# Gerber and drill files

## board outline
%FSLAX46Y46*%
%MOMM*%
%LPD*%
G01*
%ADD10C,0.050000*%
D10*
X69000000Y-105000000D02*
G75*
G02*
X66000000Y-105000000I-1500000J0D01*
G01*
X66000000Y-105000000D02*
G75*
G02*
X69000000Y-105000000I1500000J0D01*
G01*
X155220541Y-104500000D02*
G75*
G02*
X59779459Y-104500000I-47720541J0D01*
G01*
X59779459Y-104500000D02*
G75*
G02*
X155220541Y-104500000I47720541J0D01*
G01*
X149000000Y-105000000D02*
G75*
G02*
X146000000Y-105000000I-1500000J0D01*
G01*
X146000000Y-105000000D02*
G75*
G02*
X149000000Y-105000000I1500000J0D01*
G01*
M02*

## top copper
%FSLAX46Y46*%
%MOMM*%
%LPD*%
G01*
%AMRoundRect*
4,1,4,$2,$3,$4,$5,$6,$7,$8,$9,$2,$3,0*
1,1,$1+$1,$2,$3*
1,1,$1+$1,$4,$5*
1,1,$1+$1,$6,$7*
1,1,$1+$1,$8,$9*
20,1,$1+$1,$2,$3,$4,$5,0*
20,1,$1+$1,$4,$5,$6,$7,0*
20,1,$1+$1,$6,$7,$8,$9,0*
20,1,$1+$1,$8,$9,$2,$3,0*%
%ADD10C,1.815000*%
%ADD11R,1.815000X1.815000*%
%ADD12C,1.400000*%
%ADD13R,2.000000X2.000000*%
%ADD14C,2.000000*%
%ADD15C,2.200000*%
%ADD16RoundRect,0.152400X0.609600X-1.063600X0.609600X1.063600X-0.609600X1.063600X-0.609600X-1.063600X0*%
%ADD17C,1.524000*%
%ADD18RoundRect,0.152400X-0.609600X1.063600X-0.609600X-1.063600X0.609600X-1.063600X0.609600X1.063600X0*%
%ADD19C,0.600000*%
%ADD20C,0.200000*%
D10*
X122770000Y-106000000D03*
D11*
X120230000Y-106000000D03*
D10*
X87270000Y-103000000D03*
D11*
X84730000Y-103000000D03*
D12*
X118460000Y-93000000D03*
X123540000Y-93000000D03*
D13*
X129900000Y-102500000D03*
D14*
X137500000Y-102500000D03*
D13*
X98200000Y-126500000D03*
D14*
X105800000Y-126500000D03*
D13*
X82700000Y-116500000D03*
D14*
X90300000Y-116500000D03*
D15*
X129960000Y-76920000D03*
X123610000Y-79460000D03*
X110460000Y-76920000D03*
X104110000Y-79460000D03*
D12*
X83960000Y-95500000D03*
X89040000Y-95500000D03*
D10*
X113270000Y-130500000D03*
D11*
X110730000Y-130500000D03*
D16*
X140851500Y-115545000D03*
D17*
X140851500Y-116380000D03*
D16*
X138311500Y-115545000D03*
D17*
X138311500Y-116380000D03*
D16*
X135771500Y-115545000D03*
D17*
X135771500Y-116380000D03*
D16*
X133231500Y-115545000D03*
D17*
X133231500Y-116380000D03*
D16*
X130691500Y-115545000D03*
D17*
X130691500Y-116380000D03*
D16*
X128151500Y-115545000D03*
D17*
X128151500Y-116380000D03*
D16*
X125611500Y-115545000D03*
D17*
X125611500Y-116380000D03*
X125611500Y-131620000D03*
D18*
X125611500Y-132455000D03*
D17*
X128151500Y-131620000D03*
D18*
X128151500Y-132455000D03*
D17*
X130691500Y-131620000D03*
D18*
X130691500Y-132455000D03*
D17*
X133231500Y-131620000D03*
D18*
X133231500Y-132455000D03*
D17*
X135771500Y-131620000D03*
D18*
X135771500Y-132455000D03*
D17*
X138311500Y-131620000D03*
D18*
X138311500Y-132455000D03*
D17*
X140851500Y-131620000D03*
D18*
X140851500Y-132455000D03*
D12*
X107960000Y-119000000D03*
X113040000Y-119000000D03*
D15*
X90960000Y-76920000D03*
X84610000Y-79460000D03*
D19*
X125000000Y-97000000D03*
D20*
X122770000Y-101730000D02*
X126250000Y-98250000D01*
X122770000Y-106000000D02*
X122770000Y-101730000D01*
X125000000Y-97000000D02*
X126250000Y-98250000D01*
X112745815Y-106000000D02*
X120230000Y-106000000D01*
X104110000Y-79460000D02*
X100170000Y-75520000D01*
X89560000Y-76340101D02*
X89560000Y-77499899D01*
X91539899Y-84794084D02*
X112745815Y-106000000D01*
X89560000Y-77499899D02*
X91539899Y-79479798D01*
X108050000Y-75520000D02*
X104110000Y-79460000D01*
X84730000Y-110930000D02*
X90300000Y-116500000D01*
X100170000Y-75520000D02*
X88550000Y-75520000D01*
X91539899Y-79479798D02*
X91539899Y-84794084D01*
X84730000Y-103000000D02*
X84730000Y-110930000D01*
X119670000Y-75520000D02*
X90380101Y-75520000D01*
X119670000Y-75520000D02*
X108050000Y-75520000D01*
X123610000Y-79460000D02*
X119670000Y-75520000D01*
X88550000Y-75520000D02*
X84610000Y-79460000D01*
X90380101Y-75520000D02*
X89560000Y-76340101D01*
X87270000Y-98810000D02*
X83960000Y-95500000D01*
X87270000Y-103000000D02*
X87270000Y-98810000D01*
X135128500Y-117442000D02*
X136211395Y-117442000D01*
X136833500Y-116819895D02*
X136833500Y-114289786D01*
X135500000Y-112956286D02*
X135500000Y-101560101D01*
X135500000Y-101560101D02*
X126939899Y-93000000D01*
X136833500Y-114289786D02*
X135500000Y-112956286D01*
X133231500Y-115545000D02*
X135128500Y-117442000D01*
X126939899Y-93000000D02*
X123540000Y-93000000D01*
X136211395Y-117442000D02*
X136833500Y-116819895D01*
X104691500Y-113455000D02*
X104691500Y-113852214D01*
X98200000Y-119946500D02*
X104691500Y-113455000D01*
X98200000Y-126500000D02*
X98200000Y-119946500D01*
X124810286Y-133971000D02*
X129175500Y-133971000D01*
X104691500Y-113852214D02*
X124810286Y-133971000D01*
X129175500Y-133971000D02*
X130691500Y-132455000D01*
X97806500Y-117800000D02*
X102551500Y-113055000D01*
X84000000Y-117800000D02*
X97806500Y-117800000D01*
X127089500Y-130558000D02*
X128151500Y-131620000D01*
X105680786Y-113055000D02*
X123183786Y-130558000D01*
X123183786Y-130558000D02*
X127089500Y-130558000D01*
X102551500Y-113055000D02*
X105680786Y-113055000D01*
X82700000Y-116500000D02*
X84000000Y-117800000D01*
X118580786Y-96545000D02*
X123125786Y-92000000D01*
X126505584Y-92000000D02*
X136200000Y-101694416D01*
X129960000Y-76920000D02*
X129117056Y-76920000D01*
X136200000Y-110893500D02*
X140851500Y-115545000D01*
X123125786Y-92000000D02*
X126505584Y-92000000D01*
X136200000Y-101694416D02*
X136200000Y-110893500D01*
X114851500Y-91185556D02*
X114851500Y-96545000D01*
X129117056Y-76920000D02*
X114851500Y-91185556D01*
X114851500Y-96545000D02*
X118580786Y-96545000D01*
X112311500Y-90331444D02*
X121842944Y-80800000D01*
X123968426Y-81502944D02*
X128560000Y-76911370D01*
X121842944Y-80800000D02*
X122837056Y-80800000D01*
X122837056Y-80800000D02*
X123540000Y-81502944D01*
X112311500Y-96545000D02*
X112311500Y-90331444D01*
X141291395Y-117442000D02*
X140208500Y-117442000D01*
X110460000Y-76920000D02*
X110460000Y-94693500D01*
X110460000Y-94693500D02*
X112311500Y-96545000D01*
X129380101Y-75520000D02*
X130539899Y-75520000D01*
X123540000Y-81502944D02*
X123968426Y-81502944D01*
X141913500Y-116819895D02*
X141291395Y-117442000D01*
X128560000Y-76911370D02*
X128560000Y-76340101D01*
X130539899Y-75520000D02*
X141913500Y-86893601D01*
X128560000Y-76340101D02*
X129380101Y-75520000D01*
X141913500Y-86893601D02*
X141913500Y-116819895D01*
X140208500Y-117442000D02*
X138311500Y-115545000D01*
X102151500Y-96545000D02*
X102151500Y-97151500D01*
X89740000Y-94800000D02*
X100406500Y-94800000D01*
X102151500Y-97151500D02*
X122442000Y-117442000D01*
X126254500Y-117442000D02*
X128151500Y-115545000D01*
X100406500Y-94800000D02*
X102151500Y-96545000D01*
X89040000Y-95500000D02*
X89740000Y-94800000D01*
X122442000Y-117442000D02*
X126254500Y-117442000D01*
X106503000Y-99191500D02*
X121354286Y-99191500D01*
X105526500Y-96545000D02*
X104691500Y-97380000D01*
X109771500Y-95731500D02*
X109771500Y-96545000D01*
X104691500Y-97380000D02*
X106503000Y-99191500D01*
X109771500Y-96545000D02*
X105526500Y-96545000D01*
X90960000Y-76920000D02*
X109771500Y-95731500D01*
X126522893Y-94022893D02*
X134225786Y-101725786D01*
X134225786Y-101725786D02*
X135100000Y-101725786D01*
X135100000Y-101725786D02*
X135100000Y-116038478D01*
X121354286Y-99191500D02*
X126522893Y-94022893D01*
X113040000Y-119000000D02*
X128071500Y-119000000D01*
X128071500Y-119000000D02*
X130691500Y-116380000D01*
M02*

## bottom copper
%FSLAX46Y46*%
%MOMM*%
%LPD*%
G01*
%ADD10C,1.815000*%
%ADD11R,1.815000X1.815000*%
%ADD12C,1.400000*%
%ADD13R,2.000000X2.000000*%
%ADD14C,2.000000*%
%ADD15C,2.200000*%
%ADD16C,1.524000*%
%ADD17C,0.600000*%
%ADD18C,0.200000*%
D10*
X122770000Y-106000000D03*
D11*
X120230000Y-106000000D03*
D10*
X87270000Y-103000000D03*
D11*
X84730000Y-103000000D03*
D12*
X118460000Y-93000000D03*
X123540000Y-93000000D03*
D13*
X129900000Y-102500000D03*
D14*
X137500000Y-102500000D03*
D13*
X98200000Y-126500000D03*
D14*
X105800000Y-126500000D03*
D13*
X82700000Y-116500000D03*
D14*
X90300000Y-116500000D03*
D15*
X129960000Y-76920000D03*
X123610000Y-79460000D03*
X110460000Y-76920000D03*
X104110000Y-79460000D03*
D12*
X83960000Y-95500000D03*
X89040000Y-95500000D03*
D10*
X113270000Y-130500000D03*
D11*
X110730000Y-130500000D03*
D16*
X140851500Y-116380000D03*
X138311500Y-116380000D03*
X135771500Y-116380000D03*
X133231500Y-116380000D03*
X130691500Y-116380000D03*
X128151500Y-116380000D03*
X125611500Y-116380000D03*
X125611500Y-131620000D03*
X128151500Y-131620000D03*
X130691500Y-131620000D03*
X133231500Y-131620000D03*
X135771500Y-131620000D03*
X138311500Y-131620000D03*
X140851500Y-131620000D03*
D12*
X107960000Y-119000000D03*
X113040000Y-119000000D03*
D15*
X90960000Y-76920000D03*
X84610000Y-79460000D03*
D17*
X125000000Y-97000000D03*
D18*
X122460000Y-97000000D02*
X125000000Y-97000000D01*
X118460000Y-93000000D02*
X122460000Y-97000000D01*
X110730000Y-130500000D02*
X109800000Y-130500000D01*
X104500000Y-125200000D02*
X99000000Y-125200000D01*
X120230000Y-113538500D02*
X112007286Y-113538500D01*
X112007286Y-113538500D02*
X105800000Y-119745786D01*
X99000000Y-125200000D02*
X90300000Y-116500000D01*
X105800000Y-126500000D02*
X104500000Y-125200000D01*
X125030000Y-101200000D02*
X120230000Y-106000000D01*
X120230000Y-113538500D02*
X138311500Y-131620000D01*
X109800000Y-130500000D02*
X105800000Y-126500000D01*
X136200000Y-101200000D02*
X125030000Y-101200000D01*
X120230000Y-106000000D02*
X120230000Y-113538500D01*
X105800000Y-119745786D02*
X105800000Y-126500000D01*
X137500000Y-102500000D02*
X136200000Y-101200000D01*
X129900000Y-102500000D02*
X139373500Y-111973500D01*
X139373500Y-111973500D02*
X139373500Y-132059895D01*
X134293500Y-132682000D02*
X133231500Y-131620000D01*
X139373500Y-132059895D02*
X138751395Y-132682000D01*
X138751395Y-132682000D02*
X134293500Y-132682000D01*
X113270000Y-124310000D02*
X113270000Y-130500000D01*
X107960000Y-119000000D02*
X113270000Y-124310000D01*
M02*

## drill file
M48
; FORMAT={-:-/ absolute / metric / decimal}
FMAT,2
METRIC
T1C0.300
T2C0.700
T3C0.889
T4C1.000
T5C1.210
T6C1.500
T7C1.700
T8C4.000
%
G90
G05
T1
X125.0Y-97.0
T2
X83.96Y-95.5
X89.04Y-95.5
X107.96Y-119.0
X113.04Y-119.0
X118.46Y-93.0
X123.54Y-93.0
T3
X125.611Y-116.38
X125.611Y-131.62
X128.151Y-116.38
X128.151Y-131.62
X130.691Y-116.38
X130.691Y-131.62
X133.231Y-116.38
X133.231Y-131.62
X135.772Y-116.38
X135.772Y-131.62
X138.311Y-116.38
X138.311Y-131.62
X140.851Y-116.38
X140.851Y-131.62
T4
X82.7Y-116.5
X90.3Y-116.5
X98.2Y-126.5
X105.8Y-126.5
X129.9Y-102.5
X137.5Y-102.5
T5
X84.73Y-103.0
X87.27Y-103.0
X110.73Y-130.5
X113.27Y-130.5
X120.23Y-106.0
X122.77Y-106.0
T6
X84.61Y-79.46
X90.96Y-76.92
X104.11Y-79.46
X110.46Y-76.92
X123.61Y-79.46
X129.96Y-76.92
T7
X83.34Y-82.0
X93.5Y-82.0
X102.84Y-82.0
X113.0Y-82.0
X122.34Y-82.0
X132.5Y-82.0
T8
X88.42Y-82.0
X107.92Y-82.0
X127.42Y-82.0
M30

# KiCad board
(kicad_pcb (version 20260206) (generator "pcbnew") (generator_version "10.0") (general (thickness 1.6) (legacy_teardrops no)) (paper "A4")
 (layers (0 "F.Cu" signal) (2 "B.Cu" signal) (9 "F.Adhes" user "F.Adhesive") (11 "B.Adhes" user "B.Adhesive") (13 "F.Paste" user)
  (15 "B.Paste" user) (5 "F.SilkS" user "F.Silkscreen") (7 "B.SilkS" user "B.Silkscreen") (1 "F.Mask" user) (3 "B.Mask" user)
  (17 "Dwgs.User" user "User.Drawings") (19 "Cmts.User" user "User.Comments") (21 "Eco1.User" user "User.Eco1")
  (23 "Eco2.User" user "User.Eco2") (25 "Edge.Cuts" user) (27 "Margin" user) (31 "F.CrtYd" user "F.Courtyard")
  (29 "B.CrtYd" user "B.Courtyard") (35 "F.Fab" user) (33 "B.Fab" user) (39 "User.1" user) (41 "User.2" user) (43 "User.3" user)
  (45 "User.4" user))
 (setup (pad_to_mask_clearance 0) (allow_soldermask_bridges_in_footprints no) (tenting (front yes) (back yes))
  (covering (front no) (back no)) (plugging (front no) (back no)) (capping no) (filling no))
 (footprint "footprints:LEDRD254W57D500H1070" (layer "F.Cu") (at 121.5 106)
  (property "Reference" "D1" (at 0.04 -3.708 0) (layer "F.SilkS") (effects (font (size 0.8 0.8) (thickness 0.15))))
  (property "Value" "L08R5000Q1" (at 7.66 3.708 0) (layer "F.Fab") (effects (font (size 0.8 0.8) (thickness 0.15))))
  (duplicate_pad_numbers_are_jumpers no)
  (pad "A" thru_hole circle (at 1.27 0) (size 1.815 1.815) (drill 1.21) (layers "*.Cu" "*.Mask") (remove_unused_layers no)
   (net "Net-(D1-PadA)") (solder_mask_margin 0.102))
  (pad "C" thru_hole rect (at -1.27 0) (size 1.815 1.815) (drill 1.21) (layers "*.Cu" "*.Mask") (remove_unused_layers no) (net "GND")
   (solder_mask_margin 0.102)))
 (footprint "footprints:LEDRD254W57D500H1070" (layer "F.Cu") (at 86 103)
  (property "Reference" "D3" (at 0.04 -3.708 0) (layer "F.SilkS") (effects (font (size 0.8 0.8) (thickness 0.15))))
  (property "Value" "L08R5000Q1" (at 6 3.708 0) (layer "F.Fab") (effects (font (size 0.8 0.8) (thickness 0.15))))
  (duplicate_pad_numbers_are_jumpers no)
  (pad "A" thru_hole circle (at 1.27 0) (size 1.815 1.815) (drill 1.21) (layers "*.Cu" "*.Mask") (remove_unused_layers no)
   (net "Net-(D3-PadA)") (solder_mask_margin 0.102))
  (pad "C" thru_hole rect (at -1.27 0) (size 1.815 1.815) (drill 1.21) (layers "*.Cu" "*.Mask") (remove_unused_layers no) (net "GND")
   (solder_mask_margin 0.102)))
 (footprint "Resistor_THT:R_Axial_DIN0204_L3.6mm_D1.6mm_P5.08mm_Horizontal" (layer "F.Cu") (at 118.46 93)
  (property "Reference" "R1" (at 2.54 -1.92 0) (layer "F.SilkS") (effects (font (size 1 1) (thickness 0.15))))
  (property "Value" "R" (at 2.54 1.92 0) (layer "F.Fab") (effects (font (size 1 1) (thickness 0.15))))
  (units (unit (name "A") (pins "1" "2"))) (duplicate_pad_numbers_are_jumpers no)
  (pad "1" thru_hole circle (at 0 0) (size 1.4 1.4) (drill 0.7) (layers "*.Cu" "*.Mask") (remove_unused_layers no) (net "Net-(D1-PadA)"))
  (pad "2" thru_hole circle (at 5.08 0) (size 1.4 1.4) (drill 0.7) (layers "*.Cu" "*.Mask") (remove_unused_layers no)
   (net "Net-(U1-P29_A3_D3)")))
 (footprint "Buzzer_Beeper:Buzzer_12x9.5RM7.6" (layer "F.Cu") (at 129.9 102.5)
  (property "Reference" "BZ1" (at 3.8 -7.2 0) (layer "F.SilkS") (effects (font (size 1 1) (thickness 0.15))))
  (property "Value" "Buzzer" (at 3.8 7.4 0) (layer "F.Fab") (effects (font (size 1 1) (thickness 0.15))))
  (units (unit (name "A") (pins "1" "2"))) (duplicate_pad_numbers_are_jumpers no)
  (pad "1" thru_hole rect (at 0 0) (size 2 2) (drill 1) (layers "*.Cu" "*.Mask") (remove_unused_layers no) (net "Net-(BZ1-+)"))
  (pad "2" thru_hole circle (at 7.6 0) (size 2 2) (drill 1) (layers "*.Cu" "*.Mask") (remove_unused_layers no) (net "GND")))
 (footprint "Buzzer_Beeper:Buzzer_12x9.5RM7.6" (layer "F.Cu") (at 98.2 126.5)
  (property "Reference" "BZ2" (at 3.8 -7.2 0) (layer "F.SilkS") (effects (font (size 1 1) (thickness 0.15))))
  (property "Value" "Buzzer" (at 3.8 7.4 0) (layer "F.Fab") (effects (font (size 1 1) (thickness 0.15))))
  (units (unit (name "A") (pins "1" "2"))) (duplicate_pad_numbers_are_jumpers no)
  (pad "1" thru_hole rect (at 0 0) (size 2 2) (drill 1) (layers "*.Cu" "*.Mask") (remove_unused_layers no) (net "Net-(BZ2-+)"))
  (pad "2" thru_hole circle (at 7.6 0) (size 2 2) (drill 1) (layers "*.Cu" "*.Mask") (remove_unused_layers no) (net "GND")))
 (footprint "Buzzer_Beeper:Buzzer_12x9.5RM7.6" (layer "F.Cu") (at 82.7 116.5)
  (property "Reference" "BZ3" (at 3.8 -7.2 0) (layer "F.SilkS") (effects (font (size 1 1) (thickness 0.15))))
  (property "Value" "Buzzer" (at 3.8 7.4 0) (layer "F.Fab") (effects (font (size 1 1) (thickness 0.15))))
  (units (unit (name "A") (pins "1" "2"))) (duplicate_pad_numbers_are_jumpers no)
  (pad "1" thru_hole rect (at 0 0) (size 2 2) (drill 1) (layers "*.Cu" "*.Mask") (remove_unused_layers no) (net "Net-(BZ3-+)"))
  (pad "2" thru_hole circle (at 7.6 0) (size 2 2) (drill 1) (layers "*.Cu" "*.Mask") (remove_unused_layers no) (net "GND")))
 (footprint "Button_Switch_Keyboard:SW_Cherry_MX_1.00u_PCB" (layer "F.Cu") (at 129.96 76.92)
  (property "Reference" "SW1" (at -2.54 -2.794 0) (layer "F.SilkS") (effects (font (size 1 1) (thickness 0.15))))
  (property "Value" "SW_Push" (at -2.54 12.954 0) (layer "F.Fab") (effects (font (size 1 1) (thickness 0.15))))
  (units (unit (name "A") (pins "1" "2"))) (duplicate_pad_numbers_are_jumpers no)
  (pad "" np_thru_hole circle (at -7.62 5.08) (size 1.7 1.7) (drill 1.7) (layers "*.Cu" "*.Mask"))
  (pad "" np_thru_hole circle (at -2.54 5.08) (size 4 4) (drill 4) (layers "*.Cu" "*.Mask"))
  (pad "" np_thru_hole circle (at 2.54 5.08) (size 1.7 1.7) (drill 1.7) (layers "*.Cu" "*.Mask"))
  (pad "1" thru_hole circle (at 0 0) (size 2.2 2.2) (drill 1.5) (layers "*.Cu" "*.Mask") (remove_unused_layers no)
   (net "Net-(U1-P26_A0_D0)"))
  (pad "2" thru_hole circle (at -6.35 2.54) (size 2.2 2.2) (drill 1.5) (layers "*.Cu" "*.Mask") (remove_unused_layers no) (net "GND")))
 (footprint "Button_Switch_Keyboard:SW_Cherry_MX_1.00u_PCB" (layer "F.Cu") (at 110.46 76.92)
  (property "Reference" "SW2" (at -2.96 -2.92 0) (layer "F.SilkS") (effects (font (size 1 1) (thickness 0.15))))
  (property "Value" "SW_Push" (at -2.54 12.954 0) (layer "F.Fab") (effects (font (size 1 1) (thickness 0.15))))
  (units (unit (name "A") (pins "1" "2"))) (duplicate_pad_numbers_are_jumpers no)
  (pad "" np_thru_hole circle (at -7.62 5.08) (size 1.7 1.7) (drill 1.7) (layers "*.Cu" "*.Mask"))
  (pad "" np_thru_hole circle (at -2.54 5.08) (size 4 4) (drill 4) (layers "*.Cu" "*.Mask"))
  (pad "" np_thru_hole circle (at 2.54 5.08) (size 1.7 1.7) (drill 1.7) (layers "*.Cu" "*.Mask"))
  (pad "1" thru_hole circle (at 0 0) (size 2.2 2.2) (drill 1.5) (layers "*.Cu" "*.Mask") (remove_unused_layers no)
   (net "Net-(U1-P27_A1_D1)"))
  (pad "2" thru_hole circle (at -6.35 2.54) (size 2.2 2.2) (drill 1.5) (layers "*.Cu" "*.Mask") (remove_unused_layers no) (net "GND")))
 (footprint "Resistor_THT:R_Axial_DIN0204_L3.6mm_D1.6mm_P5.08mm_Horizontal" (layer "F.Cu") (at 83.96 95.5)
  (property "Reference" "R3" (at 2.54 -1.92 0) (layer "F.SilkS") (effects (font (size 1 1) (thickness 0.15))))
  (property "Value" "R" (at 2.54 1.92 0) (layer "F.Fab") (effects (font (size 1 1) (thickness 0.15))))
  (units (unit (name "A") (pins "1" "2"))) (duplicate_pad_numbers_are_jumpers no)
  (pad "1" thru_hole circle (at 0 0) (size 1.4 1.4) (drill 0.7) (layers "*.Cu" "*.Mask") (remove_unused_layers no) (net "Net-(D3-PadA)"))
  (pad "2" thru_hole circle (at 5.08 0) (size 1.4 1.4) (drill 0.7) (layers "*.Cu" "*.Mask") (remove_unused_layers no)
   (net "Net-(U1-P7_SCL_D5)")))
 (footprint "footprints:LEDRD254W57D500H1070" (layer "F.Cu") (at 112 130.5)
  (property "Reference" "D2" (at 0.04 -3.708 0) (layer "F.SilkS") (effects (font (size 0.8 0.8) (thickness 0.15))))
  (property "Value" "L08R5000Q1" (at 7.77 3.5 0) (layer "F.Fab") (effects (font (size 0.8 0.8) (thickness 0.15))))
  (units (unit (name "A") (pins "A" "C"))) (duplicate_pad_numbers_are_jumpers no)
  (pad "A" thru_hole circle (at 1.27 0) (size 1.815 1.815) (drill 1.21) (layers "*.Cu" "*.Mask") (remove_unused_layers no)
   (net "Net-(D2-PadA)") (solder_mask_margin 0.102))
  (pad "C" thru_hole rect (at -1.27 0) (size 1.815 1.815) (drill 1.21) (layers "*.Cu" "*.Mask") (remove_unused_layers no) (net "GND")
   (solder_mask_margin 0.102)))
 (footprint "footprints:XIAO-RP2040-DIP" (layer "F.Cu") (at 133.2315 124)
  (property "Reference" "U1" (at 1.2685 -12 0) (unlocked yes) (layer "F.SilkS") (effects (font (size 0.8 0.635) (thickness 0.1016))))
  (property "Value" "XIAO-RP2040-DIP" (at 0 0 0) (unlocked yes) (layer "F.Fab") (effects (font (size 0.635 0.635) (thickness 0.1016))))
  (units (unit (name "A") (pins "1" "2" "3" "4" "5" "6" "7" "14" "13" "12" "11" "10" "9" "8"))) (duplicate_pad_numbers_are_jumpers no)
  (pad "1" smd roundrect (at 7.62 -8.455 90) (size 2.432 1.524) (layers "F.Cu" "F.Mask") (roundrect_rratio 0.1) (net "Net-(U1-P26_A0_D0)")
   (thermal_bridge_angle 45))
  (pad "1" thru_hole circle (at 7.62 -7.62 90) (size 1.524 1.524) (drill 0.889) (layers "*.Cu" "*.Mask") (remove_unused_layers no)
   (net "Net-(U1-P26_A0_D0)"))
  (pad "2" smd roundrect (at 5.08 -8.455 90) (size 2.432 1.524) (layers "F.Cu" "F.Mask") (roundrect_rratio 0.1) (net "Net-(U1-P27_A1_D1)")
   (thermal_bridge_angle 45))
  (pad "2" thru_hole circle (at 5.08 -7.62 90) (size 1.524 1.524) (drill 0.889) (layers "*.Cu" "*.Mask") (remove_unused_layers no)
   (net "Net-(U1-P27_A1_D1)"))
  (pad "3" smd roundrect (at 2.54 -8.455 90) (size 2.432 1.524) (layers "F.Cu" "F.Mask") (roundrect_rratio 0.1) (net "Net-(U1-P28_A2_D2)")
   (thermal_bridge_angle 45))
  (pad "3" thru_hole circle (at 2.54 -7.62 90) (size 1.524 1.524) (drill 0.889) (layers "*.Cu" "*.Mask") (remove_unused_layers no)
   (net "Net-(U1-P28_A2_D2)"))
  (pad "4" smd roundrect (at 0 -8.455 90) (size 2.432 1.524) (layers "F.Cu" "F.Mask") (roundrect_rratio 0.1) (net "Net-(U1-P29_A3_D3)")
   (thermal_bridge_angle 45))
  (pad "4" thru_hole circle (at 0 -7.62 90) (size 1.524 1.524) (drill 0.889) (layers "*.Cu" "*.Mask") (remove_unused_layers no)
   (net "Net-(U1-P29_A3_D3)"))
  (pad "5" smd roundrect (at -2.54 -8.455 90) (size 2.432 1.524) (layers "F.Cu" "F.Mask") (roundrect_rratio 0.1) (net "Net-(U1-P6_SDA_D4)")
   (thermal_bridge_angle 45))
  (pad "5" thru_hole circle (at -2.54 -7.62 90) (size 1.524 1.524) (drill 0.889) (layers "*.Cu" "*.Mask") (remove_unused_layers no)
   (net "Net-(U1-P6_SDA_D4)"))
  (pad "6" smd roundrect (at -5.08 -8.455 90) (size 2.432 1.524) (layers "F.Cu" "F.Mask") (roundrect_rratio 0.1) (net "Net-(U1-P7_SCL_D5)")
   (thermal_bridge_angle 45))
  (pad "6" thru_hole circle (at -5.08 -7.62 90) (size 1.524 1.524) (drill 0.889) (layers "*.Cu" "*.Mask") (remove_unused_layers no)
   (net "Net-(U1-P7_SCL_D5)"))
  (pad "7" smd roundrect (at -7.62 -8.455 90) (size 2.432 1.524) (layers "F.Cu" "F.Mask") (roundrect_rratio 0.1)
   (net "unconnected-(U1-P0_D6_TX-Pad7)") (thermal_bridge_angle 45))
  (pad "7" thru_hole circle (at -7.62 -7.62 90) (size 1.524 1.524) (drill 0.889) (layers "*.Cu" "*.Mask") (remove_unused_layers no)
   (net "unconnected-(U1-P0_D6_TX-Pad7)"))
  (pad "8" thru_hole circle (at -7.62 7.62 270) (size 1.524 1.524) (drill 0.889) (layers "*.Cu" "*.Mask") (remove_unused_layers no)
   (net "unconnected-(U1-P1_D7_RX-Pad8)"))
  (pad "8" smd roundrect (at -7.62 8.455 270) (size 2.432 1.524) (layers "F.Cu" "F.Mask") (roundrect_rratio 0.1)
   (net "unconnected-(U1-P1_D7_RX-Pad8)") (thermal_bridge_angle 45))
  (pad "9" thru_hole circle (at -5.08 7.62 270) (size 1.524 1.524) (drill 0.889) (layers "*.Cu" "*.Mask") (remove_unused_layers no)
   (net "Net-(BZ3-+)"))
  (pad "9" smd roundrect (at -5.08 8.455 270) (size 2.432 1.524) (layers "F.Cu" "F.Mask") (roundrect_rratio 0.1) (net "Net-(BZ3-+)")
   (thermal_bridge_angle 45))
  (pad "10" thru_hole circle (at -2.54 7.62 270) (size 1.524 1.524) (drill 0.889) (layers "*.Cu" "*.Mask") (remove_unused_layers no)
   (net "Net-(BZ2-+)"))
  (pad "10" smd roundrect (at -2.54 8.455 270) (size 2.432 1.524) (layers "F.Cu" "F.Mask") (roundrect_rratio 0.1) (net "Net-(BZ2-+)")
   (thermal_bridge_angle 45))
  (pad "11" thru_hole circle (at 0 7.62 270) (size 1.524 1.524) (drill 0.889) (layers "*.Cu" "*.Mask") (remove_unused_layers no)
   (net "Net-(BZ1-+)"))
  (pad "11" smd roundrect (at 0 8.455 270) (size 2.432 1.524) (layers "F.Cu" "F.Mask") (roundrect_rratio 0.1) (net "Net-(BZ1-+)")
   (thermal_bridge_angle 45))
  (pad "12" thru_hole circle (at 2.54 7.62 270) (size 1.524 1.524) (drill 0.889) (layers "*.Cu" "*.Mask") (remove_unused_layers no)
   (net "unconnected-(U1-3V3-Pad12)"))
  (pad "12" smd roundrect (at 2.54 8.455 270) (size 2.432 1.524) (layers "F.Cu" "F.Mask") (roundrect_rratio 0.1)
   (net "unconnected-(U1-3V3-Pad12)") (thermal_bridge_angle 45))
  (pad "13" thru_hole circle (at 5.08 7.62 270) (size 1.524 1.524) (drill 0.889) (layers "*.Cu" "*.Mask") (remove_unused_layers no)
   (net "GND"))
  (pad "13" smd roundrect (at 5.08 8.455 270) (size 2.432 1.524) (layers "F.Cu" "F.Mask") (roundrect_rratio 0.1) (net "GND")
   (thermal_bridge_angle 45))
  (pad "14" thru_hole circle (at 7.62 7.62 270) (size 1.524 1.524) (drill 0.889) (layers "*.Cu" "*.Mask") (remove_unused_layers no)
   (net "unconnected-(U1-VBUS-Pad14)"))
  (pad "14" smd roundrect (at 7.62 8.455 270) (size 2.432 1.524) (layers "F.Cu" "F.Mask") (roundrect_rratio 0.1)
   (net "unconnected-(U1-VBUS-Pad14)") (thermal_bridge_angle 45)))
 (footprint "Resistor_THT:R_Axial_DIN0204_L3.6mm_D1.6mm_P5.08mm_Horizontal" (layer "F.Cu") (at 107.96 119)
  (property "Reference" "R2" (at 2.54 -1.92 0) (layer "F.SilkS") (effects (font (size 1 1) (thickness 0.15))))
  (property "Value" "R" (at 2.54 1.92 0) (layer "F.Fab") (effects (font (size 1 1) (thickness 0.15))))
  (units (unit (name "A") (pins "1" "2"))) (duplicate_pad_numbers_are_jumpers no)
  (pad "1" thru_hole circle (at 0 0) (size 1.4 1.4) (drill 0.7) (layers "*.Cu" "*.Mask") (remove_unused_layers no) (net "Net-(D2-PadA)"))
  (pad "2" thru_hole circle (at 5.08 0) (size 1.4 1.4) (drill 0.7) (layers "*.Cu" "*.Mask") (remove_unused_layers no)
   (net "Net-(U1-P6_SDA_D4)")))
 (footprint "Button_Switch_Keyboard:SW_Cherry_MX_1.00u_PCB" (layer "F.Cu") (at 90.96 76.92)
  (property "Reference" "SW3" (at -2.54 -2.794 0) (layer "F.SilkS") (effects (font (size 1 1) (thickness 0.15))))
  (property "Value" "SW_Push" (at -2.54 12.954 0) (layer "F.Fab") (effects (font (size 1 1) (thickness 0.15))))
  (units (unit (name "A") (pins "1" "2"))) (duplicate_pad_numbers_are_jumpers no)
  (pad "" np_thru_hole circle (at -7.62 5.08) (size 1.7 1.7) (drill 1.7) (layers "*.Cu" "*.Mask"))
  (pad "" np_thru_hole circle (at -2.54 5.08) (size 4 4) (drill 4) (layers "*.Cu" "*.Mask"))
  (pad "" np_thru_hole circle (at 2.54 5.08) (size 1.7 1.7) (drill 1.7) (layers "*.Cu" "*.Mask"))
  (pad "1" thru_hole circle (at 0 0) (size 2.2 2.2) (drill 1.5) (layers "*.Cu" "*.Mask") (remove_unused_layers no)
   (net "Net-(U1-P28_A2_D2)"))
  (pad "2" thru_hole circle (at -6.35 2.54) (size 2.2 2.2) (drill 1.5) (layers "*.Cu" "*.Mask") (remove_unused_layers no) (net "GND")))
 (gr_circle (center 67.5 105) (end 66 105) (stroke (width 0.05) (type default)) (fill no) (layer "Edge.Cuts"))
 (gr_circle (center 107.5 104.5) (end 80 65.5) (stroke (width 0.05) (type default)) (fill no) (layer "Edge.Cuts"))
 (gr_circle (center 147.5 105) (end 149 105) (stroke (width 0.05) (type default)) (fill no) (layer "Edge.Cuts"))
 (segment (start 122.77 101.73) (end 126.25 98.25) (width 0.2) (layer "F.Cu") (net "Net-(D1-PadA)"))
 (segment (start 122.77 106) (end 122.77 101.73) (width 0.2) (layer "F.Cu") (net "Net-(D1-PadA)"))
 (segment (start 125 97) (end 126.25 98.25) (width 0.2) (layer "F.Cu") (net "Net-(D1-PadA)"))
 (via (at 125 97) (size 0.6) (drill 0.3) (layers "F.Cu" "B.Cu") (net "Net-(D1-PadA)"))
 (segment (start 122.46 97) (end 125 97) (width 0.2) (layer "B.Cu") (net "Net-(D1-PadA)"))
 (segment (start 118.46 93) (end 122.46 97) (width 0.2) (layer "B.Cu") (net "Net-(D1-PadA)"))
 (segment (start 112.745815 106) (end 120.23 106) (width 0.2) (layer "F.Cu") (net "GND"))
 (segment (start 104.11 79.46) (end 100.17 75.52) (width 0.2) (layer "F.Cu") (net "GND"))
 (segment (start 89.56 76.340101) (end 89.56 77.499899) (width 0.2) (layer "F.Cu") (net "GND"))
 (segment (start 91.539899 84.794084) (end 112.745815 106) (width 0.2) (layer "F.Cu") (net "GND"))
 (segment (start 89.56 77.499899) (end 91.539899 79.479798) (width 0.2) (layer "F.Cu") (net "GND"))
 (segment (start 108.05 75.52) (end 104.11 79.46) (width 0.2) (layer "F.Cu") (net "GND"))
 (segment (start 84.73 110.93) (end 90.3 116.5) (width 0.2) (layer "F.Cu") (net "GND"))
 (segment (start 100.17 75.52) (end 88.55 75.52) (width 0.2) (layer "F.Cu") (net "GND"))
 (segment (start 91.539899 79.479798) (end 91.539899 84.794084) (width 0.2) (layer "F.Cu") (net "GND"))
 (segment (start 84.73 103) (end 84.73 110.93) (width 0.2) (layer "F.Cu") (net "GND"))
 (segment (start 119.67 75.52) (end 90.380101 75.52) (width 0.2) (layer "F.Cu") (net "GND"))
 (segment (start 119.67 75.52) (end 108.05 75.52) (width 0.2) (layer "F.Cu") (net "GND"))
 (segment (start 123.61 79.46) (end 119.67 75.52) (width 0.2) (layer "F.Cu") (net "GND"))
 (segment (start 88.55 75.52) (end 84.61 79.46) (width 0.2) (layer "F.Cu") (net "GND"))
 (segment (start 90.380101 75.52) (end 89.56 76.340101) (width 0.2) (layer "F.Cu") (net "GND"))
 (segment (start 110.73 130.5) (end 109.8 130.5) (width 0.2) (layer "B.Cu") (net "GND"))
 (segment (start 104.5 125.2) (end 99 125.2) (width 0.2) (layer "B.Cu") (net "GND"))
 (segment (start 120.23 113.5385) (end 112.007286 113.5385) (width 0.2) (layer "B.Cu") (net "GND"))
 (segment (start 112.007286 113.5385) (end 105.8 119.745786) (width 0.2) (layer "B.Cu") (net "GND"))
 (segment (start 99 125.2) (end 90.3 116.5) (width 0.2) (layer "B.Cu") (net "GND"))
 (segment (start 105.8 126.5) (end 104.5 125.2) (width 0.2) (layer "B.Cu") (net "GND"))
 (segment (start 125.03 101.2) (end 120.23 106) (width 0.2) (layer "B.Cu") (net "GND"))
 (segment (start 120.23 113.5385) (end 138.3115 131.62) (width 0.2) (layer "B.Cu") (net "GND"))
 (segment (start 109.8 130.5) (end 105.8 126.5) (width 0.2) (layer "B.Cu") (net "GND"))
 (segment (start 136.2 101.2) (end 125.03 101.2) (width 0.2) (layer "B.Cu") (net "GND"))
 (segment (start 120.23 106) (end 120.23 113.5385) (width 0.2) (layer "B.Cu") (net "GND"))
 (segment (start 105.8 119.745786) (end 105.8 126.5) (width 0.2) (layer "B.Cu") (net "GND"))
 (segment (start 137.5 102.5) (end 136.2 101.2) (width 0.2) (layer "B.Cu") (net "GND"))
 (segment (start 87.27 98.81) (end 83.96 95.5) (width 0.2) (layer "F.Cu") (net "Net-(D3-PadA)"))
 (segment (start 87.27 103) (end 87.27 98.81) (width 0.2) (layer "F.Cu") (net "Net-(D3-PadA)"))
 (segment (start 135.1285 117.442) (end 136.211395 117.442) (width 0.2) (layer "F.Cu") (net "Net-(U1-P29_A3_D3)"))
 (segment (start 136.8335 116.819895) (end 136.8335 114.289786) (width 0.2) (layer "F.Cu") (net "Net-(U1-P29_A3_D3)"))
 (segment (start 135.5 112.956286) (end 135.5 101.560101) (width 0.2) (layer "F.Cu") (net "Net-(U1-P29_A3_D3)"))
 (segment (start 135.5 101.560101) (end 126.939899 93) (width 0.2) (layer "F.Cu") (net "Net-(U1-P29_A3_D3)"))
 (segment (start 136.8335 114.289786) (end 135.5 112.956286) (width 0.2) (layer "F.Cu") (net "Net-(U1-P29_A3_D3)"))
 (segment (start 133.2315 115.545) (end 135.1285 117.442) (width 0.2) (layer "F.Cu") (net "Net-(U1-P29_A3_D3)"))
 (segment (start 126.939899 93) (end 123.54 93) (width 0.2) (layer "F.Cu") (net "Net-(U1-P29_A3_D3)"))
 (segment (start 136.211395 117.442) (end 136.8335 116.819895) (width 0.2) (layer "F.Cu") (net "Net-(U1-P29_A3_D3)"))
 (segment (start 129.9 102.5) (end 139.3735 111.9735) (width 0.2) (layer "B.Cu") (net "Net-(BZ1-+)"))
 (segment (start 139.3735 111.9735) (end 139.3735 132.059895) (width 0.2) (layer "B.Cu") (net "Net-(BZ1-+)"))
 (segment (start 134.2935 132.682) (end 133.2315 131.62) (width 0.2) (layer "B.Cu") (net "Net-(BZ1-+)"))
 (segment (start 139.3735 132.059895) (end 138.751395 132.682) (width 0.2) (layer "B.Cu") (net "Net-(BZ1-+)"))
 (segment (start 138.751395 132.682) (end 134.2935 132.682) (width 0.2) (layer "B.Cu") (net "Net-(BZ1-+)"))
 (segment (start 104.6915 113.455) (end 104.6915 113.852214) (width 0.2) (layer "F.Cu") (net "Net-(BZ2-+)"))
 (segment (start 98.2 119.9465) (end 104.6915 113.455) (width 0.2) (layer "F.Cu") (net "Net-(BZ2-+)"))
 (segment (start 98.2 126.5) (end 98.2 119.9465) (width 0.2) (layer "F.Cu") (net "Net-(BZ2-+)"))
 (segment (start 124.810286 133.971) (end 129.1755 133.971) (width 0.2) (layer "F.Cu") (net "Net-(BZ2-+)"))
 (segment (start 104.6915 113.852214) (end 124.810286 133.971) (width 0.2) (layer "F.Cu") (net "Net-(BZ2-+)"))
 (segment (start 129.1755 133.971) (end 130.6915 132.455) (width 0.2) (layer "F.Cu") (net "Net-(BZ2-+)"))
 (segment (start 97.8065 117.8) (end 102.5515 113.055) (width 0.2) (layer "F.Cu") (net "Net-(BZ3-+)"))
 (segment (start 84 117.8) (end 97.8065 117.8) (width 0.2) (layer "F.Cu") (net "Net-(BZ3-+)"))
 (segment (start 127.0895 130.558) (end 128.1515 131.62) (width 0.2) (layer "F.Cu") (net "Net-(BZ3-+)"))
 (segment (start 105.680786 113.055) (end 123.183786 130.558) (width 0.2) (layer "F.Cu") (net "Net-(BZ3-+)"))
 (segment (start 123.183786 130.558) (end 127.0895 130.558) (width 0.2) (layer "F.Cu") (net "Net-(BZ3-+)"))
 (segment (start 102.5515 113.055) (end 105.680786 113.055) (width 0.2) (layer "F.Cu") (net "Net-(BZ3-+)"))
 (segment (start 82.7 116.5) (end 84 117.8) (width 0.2) (layer "F.Cu") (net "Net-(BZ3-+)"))
 (segment (start 118.580786 96.545) (end 123.125786 92) (width 0.2) (layer "F.Cu") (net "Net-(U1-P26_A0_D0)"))
 (segment (start 126.505584 92) (end 136.2 101.694416) (width 0.2) (layer "F.Cu") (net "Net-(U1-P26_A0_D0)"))
 (segment (start 129.96 76.92) (end 129.117056 76.92) (width 0.2) (layer "F.Cu") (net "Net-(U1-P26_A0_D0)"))
 (segment (start 136.2 110.8935) (end 140.8515 115.545) (width 0.2) (layer "F.Cu") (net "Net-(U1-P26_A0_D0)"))
 (segment (start 123.125786 92) (end 126.505584 92) (width 0.2) (layer "F.Cu") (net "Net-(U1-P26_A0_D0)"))
 (segment (start 136.2 101.694416) (end 136.2 110.8935) (width 0.2) (layer "F.Cu") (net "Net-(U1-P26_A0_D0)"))
 (segment (start 114.8515 91.185556) (end 114.8515 96.545) (width 0.2) (layer "F.Cu") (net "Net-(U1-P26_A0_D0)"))
 (segment (start 129.117056 76.92) (end 114.8515 91.185556) (width 0.2) (layer "F.Cu") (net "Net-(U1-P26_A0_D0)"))
 (segment (start 114.8515 96.545) (end 118.580786 96.545) (width 0.2) (layer "F.Cu") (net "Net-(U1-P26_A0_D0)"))
 (segment (start 112.3115 90.331444) (end 121.842944 80.8) (width 0.2) (layer "F.Cu") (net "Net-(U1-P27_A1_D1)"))
 (segment (start 123.968426 81.502944) (end 128.56 76.91137) (width 0.2) (layer "F.Cu") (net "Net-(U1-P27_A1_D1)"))
 (segment (start 121.842944 80.8) (end 122.837056 80.8) (width 0.2) (layer "F.Cu") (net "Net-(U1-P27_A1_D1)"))
 (segment (start 122.837056 80.8) (end 123.54 81.502944) (width 0.2) (layer "F.Cu") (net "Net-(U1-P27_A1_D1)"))
 (segment (start 112.3115 96.545) (end 112.3115 90.331444) (width 0.2) (layer "F.Cu") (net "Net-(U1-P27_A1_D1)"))
 (segment (start 141.291395 117.442) (end 140.2085 117.442) (width 0.2) (layer "F.Cu") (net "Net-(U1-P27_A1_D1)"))
 (segment (start 110.46 76.92) (end 110.46 94.6935) (width 0.2) (layer "F.Cu") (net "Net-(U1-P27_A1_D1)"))
 (segment (start 110.46 94.6935) (end 112.3115 96.545) (width 0.2) (layer "F.Cu") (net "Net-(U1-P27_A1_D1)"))
 (segment (start 129.380101 75.52) (end 130.539899 75.52) (width 0.2) (layer "F.Cu") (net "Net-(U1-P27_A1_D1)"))
 (segment (start 123.54 81.502944) (end 123.968426 81.502944) (width 0.2) (layer "F.Cu") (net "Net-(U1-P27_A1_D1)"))
 (segment (start 141.9135 116.819895) (end 141.291395 117.442) (width 0.2) (layer "F.Cu") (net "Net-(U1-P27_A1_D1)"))
 (segment (start 128.56 76.91137) (end 128.56 76.340101) (width 0.2) (layer "F.Cu") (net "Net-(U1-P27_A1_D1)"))
 (segment (start 130.539899 75.52) (end 141.9135 86.893601) (width 0.2) (layer "F.Cu") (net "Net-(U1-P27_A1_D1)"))
 (segment (start 128.56 76.340101) (end 129.380101 75.52) (width 0.2) (layer "F.Cu") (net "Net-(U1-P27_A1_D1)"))
 (segment (start 141.9135 86.893601) (end 141.9135 116.819895) (width 0.2) (layer "F.Cu") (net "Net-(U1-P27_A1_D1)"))
 (segment (start 140.2085 117.442) (end 138.3115 115.545) (width 0.2) (layer "F.Cu") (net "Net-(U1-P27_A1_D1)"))
 (segment (start 102.1515 96.545) (end 102.1515 97.1515) (width 0.2) (layer "F.Cu") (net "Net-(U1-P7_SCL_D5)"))
 (segment (start 89.74 94.8) (end 100.4065 94.8) (width 0.2) (layer "F.Cu") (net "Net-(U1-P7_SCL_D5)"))
 (segment (start 102.1515 97.1515) (end 122.442 117.442) (width 0.2) (layer "F.Cu") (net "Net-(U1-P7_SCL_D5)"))
 (segment (start 126.2545 117.442) (end 128.1515 115.545) (width 0.2) (layer "F.Cu") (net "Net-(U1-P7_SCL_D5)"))
 (segment (start 100.4065 94.8) (end 102.1515 96.545) (width 0.2) (layer "F.Cu") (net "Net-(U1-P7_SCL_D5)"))
 (segment (start 89.04 95.5) (end 89.74 94.8) (width 0.2) (layer "F.Cu") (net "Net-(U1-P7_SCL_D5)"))
 (segment (start 122.442 117.442) (end 126.2545 117.442) (width 0.2) (layer "F.Cu") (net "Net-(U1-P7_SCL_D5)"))
 (segment (start 113.27 124.31) (end 113.27 130.5) (width 0.2) (layer "B.Cu") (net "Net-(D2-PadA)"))
 (segment (start 107.96 119) (end 113.27 124.31) (width 0.2) (layer "B.Cu") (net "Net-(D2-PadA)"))
 (segment (start 106.503 99.1915) (end 121.354286 99.1915) (width 0.2) (layer "F.Cu") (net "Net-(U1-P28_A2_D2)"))
 (segment (start 105.5265 96.545) (end 104.6915 97.38) (width 0.2) (layer "F.Cu") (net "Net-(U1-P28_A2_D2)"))
 (segment (start 109.7715 95.7315) (end 109.7715 96.545) (width 0.2) (layer "F.Cu") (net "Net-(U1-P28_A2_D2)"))
 (segment (start 104.6915 97.38) (end 106.503 99.1915) (width 0.2) (layer "F.Cu") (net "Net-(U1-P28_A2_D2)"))
 (segment (start 109.7715 96.545) (end 105.5265 96.545) (width 0.2) (layer "F.Cu") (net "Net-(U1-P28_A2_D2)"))
 (segment (start 90.96 76.92) (end 109.7715 95.7315) (width 0.2) (layer "F.Cu") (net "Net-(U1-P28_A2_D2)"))
 (segment (start 126.522893 94.022893) (end 134.225786 101.725786) (width 0.2) (layer "F.Cu") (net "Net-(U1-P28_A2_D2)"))
 (segment (start 134.225786 101.725786) (end 135.1 101.725786) (width 0.2) (layer "F.Cu") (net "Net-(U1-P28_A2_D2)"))
 (segment (start 135.1 101.725786) (end 135.1 116.038478) (width 0.2) (layer "F.Cu") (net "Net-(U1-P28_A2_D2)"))
 (segment (start 121.354286 99.1915) (end 126.522893 94.022893) (width 0.2) (layer "F.Cu") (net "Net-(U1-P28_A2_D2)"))
 (segment (start 113.04 119) (end 128.0715 119) (width 0.2) (layer "F.Cu") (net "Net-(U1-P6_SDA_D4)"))
 (segment (start 128.0715 119) (end 130.6915 116.38) (width 0.2) (layer "F.Cu") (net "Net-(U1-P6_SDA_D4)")))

